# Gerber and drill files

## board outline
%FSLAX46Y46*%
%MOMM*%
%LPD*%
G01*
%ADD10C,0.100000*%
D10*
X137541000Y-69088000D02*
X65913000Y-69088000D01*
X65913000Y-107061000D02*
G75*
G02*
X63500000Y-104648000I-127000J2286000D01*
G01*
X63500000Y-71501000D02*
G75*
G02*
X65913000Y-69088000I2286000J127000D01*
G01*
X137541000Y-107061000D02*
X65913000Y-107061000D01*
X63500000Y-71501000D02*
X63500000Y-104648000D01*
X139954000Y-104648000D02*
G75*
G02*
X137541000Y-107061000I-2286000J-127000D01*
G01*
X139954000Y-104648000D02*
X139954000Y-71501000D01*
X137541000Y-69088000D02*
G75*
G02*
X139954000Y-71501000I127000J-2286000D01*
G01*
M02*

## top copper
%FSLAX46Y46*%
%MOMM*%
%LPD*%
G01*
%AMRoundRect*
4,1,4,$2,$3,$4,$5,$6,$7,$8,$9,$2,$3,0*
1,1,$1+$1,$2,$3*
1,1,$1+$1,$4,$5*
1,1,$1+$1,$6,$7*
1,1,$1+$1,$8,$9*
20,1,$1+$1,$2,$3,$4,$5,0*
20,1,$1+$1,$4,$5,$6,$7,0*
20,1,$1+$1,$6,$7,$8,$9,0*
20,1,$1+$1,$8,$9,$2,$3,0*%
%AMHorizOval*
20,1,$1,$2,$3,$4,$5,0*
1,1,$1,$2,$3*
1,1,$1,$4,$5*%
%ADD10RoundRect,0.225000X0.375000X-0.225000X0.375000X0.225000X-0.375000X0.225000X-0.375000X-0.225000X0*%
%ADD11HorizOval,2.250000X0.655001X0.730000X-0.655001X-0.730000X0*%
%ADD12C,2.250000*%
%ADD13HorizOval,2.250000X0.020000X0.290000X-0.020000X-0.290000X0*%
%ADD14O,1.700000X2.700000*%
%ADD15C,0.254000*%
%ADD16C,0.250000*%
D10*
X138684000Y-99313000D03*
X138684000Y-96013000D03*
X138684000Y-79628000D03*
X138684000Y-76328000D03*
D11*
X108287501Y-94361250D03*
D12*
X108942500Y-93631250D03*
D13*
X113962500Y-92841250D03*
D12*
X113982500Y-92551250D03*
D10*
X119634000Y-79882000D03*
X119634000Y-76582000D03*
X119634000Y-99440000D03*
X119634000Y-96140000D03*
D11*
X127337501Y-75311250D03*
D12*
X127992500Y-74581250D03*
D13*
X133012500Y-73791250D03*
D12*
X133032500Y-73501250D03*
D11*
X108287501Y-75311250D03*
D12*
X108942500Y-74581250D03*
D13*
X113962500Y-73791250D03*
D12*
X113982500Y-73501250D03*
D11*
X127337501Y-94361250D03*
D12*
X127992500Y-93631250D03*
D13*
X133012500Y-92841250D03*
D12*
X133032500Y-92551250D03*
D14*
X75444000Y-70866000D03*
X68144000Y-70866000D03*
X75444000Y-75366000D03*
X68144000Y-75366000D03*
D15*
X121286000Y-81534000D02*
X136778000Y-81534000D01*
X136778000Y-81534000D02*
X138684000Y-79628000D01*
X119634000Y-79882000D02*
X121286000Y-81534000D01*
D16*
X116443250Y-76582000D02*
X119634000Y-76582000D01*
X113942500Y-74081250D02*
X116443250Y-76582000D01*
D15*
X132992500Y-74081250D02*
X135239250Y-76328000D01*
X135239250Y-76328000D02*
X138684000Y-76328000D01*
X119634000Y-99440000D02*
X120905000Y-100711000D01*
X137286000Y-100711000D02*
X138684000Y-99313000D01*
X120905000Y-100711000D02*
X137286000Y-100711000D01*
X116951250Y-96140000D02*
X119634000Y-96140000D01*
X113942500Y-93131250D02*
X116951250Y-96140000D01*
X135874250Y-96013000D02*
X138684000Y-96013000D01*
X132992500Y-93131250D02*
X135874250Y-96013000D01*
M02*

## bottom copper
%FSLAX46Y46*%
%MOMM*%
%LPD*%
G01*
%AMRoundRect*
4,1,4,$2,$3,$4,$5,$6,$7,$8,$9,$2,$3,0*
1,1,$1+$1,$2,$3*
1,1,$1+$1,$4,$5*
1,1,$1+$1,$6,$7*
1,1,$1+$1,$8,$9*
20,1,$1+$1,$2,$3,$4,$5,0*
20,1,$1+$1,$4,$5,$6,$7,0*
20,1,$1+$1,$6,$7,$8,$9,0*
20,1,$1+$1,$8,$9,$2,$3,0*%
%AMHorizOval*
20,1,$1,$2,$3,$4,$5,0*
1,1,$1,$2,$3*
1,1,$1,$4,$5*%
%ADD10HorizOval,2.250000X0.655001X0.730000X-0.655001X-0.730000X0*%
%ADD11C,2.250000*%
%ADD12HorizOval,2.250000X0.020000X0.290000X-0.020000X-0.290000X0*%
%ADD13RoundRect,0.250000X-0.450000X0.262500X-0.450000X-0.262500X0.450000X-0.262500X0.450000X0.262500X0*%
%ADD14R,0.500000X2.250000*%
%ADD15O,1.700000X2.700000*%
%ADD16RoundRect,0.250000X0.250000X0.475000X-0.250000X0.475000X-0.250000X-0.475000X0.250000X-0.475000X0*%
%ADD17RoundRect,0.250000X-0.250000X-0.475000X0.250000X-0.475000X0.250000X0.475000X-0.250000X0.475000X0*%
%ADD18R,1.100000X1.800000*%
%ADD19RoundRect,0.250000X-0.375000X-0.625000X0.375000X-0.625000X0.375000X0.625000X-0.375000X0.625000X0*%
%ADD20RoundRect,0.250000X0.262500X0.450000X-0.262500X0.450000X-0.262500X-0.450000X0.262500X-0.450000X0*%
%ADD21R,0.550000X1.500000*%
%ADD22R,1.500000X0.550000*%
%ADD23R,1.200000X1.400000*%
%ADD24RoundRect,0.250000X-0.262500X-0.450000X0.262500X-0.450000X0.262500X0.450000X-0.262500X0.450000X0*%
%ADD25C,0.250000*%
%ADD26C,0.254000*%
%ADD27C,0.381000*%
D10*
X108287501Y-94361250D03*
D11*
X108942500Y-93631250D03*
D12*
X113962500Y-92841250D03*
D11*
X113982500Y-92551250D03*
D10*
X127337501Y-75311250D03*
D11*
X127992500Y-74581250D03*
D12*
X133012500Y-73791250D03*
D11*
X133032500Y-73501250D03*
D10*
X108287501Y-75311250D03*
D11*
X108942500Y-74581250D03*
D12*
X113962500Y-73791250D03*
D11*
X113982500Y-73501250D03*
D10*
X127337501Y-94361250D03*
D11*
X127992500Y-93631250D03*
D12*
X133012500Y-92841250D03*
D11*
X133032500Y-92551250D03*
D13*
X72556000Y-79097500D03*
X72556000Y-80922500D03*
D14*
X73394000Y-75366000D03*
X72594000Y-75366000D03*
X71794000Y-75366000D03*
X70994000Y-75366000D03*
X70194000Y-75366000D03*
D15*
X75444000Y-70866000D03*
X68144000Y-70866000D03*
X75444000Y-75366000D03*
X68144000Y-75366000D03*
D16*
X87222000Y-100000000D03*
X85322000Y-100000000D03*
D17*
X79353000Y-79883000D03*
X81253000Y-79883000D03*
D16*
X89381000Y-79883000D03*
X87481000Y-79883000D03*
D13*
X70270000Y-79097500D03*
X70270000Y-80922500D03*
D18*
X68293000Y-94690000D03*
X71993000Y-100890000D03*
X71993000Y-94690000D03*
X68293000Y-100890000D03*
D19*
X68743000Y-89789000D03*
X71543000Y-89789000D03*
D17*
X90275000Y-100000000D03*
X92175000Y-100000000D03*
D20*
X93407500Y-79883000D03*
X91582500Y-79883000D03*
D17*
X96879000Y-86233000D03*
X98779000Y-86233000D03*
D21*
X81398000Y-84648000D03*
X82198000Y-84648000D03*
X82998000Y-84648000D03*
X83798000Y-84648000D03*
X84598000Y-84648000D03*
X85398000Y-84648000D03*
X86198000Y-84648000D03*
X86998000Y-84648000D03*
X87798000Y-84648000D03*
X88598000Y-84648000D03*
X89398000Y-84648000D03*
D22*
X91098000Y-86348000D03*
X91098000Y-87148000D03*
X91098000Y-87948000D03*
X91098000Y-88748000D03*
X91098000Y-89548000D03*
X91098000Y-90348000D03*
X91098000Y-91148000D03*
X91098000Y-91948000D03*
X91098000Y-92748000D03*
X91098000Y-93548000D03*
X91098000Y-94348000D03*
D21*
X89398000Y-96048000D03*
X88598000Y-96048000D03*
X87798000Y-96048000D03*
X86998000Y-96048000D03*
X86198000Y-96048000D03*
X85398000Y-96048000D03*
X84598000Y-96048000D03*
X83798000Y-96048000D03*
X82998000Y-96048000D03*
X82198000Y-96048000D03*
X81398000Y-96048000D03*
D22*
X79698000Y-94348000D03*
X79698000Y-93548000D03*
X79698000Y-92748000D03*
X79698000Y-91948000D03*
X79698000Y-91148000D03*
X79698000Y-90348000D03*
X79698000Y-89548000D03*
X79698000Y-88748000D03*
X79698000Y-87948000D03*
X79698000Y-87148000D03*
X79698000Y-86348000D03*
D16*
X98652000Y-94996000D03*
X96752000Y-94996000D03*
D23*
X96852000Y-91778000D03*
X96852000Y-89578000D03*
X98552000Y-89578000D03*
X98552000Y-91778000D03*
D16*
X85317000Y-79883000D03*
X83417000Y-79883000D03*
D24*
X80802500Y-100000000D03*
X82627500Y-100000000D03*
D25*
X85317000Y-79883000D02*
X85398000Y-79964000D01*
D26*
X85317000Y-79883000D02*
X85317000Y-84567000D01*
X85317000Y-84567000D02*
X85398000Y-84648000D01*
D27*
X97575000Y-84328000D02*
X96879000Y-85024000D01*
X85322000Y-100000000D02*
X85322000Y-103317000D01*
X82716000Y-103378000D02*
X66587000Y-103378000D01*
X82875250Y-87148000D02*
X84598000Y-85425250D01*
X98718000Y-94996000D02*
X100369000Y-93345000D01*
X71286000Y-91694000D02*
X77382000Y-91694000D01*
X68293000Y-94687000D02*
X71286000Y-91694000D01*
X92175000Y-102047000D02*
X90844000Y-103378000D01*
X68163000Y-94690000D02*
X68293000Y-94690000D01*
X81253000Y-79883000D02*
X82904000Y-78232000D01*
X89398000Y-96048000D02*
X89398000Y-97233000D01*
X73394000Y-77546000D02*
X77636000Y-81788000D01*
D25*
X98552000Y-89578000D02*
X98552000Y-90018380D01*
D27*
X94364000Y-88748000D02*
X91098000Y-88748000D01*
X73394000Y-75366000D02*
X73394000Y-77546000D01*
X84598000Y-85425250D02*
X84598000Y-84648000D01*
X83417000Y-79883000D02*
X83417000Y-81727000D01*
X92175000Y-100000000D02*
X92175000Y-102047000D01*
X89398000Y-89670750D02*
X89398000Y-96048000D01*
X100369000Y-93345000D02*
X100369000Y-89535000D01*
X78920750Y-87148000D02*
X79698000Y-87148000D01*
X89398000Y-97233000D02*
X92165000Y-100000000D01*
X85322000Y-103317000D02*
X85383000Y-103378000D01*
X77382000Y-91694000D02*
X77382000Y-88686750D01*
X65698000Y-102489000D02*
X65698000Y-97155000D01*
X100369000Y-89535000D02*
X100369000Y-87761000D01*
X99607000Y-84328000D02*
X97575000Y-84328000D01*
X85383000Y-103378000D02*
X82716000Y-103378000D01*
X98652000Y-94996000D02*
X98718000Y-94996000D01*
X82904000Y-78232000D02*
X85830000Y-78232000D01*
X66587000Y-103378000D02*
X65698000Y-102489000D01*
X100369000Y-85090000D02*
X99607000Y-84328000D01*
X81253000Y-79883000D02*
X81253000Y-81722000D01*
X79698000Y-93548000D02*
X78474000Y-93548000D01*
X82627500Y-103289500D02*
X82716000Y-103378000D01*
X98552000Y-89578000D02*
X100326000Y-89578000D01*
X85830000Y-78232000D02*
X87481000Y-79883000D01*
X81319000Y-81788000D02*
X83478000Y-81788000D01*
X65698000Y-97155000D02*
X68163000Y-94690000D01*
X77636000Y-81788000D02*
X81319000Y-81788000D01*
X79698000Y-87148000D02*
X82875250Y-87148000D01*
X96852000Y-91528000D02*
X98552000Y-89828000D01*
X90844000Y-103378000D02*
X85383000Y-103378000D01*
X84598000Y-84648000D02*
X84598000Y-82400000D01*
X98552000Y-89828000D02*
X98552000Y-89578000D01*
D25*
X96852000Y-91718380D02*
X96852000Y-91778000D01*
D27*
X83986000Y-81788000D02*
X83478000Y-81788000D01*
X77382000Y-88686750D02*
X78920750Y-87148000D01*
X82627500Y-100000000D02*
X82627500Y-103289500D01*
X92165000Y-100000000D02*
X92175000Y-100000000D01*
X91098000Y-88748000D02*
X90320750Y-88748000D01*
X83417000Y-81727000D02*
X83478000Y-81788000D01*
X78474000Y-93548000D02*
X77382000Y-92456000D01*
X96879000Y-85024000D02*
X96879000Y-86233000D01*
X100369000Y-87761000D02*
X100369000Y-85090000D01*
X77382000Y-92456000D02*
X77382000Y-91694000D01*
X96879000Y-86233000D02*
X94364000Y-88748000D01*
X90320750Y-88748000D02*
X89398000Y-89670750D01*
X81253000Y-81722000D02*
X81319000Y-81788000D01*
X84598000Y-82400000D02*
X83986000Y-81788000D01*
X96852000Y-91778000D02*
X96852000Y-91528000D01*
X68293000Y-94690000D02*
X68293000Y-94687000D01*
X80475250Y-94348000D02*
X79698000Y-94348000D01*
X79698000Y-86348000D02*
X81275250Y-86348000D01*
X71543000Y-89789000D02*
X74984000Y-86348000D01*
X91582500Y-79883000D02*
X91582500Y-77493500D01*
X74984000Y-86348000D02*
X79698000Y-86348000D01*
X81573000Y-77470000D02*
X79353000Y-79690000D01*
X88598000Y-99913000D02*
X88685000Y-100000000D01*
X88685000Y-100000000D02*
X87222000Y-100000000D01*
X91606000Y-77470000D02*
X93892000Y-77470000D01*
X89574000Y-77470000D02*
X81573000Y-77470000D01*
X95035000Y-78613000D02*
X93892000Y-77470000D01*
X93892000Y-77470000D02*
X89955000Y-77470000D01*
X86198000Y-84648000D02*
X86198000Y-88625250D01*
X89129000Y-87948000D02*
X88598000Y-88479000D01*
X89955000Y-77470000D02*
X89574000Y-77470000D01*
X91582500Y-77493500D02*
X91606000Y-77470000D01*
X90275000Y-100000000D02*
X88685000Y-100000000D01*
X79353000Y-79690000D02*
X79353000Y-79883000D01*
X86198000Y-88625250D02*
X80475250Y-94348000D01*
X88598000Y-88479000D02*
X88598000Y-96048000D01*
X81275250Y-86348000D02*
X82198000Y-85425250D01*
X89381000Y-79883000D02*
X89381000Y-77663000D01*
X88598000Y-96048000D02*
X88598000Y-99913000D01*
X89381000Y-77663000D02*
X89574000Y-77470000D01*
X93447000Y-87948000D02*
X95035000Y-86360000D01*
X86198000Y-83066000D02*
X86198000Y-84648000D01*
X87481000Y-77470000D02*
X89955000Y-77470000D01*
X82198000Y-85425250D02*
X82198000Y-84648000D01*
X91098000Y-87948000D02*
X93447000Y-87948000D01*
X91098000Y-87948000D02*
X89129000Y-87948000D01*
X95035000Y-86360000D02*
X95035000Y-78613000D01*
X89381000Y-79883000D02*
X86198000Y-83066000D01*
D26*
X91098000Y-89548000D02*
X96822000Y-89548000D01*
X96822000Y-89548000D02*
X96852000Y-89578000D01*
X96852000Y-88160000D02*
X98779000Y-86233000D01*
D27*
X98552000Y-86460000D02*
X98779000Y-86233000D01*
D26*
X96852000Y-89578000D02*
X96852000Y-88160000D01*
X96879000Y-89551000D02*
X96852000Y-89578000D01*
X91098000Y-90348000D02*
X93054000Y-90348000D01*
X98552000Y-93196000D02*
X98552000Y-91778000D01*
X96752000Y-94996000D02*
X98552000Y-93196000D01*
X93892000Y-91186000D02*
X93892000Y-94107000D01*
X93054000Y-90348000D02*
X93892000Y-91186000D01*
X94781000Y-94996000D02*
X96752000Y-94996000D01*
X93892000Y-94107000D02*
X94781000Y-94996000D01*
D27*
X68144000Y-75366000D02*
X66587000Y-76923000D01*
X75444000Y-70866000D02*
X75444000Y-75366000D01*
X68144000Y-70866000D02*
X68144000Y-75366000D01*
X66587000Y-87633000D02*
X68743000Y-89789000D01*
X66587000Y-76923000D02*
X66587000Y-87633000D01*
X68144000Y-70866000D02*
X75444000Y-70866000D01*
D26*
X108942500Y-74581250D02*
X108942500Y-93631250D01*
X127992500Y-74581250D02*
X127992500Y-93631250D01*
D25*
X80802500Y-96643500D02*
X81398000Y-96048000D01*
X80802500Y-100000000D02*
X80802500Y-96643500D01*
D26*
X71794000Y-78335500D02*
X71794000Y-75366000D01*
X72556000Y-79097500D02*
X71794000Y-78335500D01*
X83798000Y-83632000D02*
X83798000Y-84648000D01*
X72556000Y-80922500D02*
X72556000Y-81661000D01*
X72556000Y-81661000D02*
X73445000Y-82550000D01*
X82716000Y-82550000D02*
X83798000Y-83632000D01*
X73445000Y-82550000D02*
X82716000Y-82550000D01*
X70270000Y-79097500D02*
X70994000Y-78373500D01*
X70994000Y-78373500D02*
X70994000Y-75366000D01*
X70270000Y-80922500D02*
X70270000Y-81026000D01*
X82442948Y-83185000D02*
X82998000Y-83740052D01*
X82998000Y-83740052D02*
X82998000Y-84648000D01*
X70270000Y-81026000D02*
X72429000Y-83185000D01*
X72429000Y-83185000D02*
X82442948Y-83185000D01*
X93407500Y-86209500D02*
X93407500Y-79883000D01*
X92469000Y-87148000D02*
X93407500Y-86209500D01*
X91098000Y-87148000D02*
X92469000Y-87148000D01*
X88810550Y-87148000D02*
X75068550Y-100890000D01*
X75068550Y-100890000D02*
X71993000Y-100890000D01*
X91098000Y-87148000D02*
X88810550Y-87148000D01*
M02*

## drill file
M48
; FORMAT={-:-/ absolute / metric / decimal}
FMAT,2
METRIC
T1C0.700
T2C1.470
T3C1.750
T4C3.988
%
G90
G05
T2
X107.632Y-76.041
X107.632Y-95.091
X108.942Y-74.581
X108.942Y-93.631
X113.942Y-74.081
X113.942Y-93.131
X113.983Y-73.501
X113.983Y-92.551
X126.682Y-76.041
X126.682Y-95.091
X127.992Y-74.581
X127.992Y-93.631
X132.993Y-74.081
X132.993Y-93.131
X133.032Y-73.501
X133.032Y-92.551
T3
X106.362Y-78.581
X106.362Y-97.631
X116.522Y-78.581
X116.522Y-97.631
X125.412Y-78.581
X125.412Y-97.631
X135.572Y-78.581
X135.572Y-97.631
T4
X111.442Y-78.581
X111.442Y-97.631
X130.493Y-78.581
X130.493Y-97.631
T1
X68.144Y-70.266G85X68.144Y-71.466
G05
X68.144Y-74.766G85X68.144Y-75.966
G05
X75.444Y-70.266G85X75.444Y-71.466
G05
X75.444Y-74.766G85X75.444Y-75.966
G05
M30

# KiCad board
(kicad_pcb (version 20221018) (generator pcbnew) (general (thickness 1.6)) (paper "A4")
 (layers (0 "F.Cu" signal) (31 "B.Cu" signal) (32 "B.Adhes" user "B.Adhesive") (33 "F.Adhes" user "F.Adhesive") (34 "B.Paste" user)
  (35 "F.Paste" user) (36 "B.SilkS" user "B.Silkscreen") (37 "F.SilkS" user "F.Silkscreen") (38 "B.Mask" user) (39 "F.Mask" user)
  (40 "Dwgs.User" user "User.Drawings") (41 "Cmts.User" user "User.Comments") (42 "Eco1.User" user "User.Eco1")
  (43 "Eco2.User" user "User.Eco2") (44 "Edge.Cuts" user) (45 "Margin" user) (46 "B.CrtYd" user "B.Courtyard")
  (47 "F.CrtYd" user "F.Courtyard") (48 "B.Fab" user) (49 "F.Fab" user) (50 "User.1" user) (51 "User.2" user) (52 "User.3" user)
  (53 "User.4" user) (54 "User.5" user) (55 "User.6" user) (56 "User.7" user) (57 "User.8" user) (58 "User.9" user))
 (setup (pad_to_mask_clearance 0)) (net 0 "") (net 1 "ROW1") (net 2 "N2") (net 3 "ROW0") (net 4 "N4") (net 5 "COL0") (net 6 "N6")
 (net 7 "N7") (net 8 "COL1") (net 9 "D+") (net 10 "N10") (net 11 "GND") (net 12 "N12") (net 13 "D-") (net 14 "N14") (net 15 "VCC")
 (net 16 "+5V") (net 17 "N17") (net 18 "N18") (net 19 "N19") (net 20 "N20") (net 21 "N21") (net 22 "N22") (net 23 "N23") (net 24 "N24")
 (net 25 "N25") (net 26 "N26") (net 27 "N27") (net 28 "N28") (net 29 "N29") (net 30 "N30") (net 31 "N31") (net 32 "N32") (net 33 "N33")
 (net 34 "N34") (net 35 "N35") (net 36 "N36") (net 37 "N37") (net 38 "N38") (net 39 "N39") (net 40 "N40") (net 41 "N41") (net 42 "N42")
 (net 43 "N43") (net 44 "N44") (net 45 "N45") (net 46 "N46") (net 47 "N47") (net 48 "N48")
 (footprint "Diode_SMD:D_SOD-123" (layer "F.Cu") (at 138.684 97.663 90)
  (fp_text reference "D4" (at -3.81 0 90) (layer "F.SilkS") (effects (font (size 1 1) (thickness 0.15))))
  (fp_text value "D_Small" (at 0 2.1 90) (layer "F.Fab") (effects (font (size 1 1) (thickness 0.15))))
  (pad "1" smd roundrect (at -1.65 0 90) (size 0.9 1.2) (layers "F.Cu" "F.Paste" "F.Mask") (roundrect_rratio 0.25) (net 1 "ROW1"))
  (pad "2" smd roundrect (at 1.65 0 90) (size 0.9 1.2) (layers "F.Cu" "F.Paste" "F.Mask") (roundrect_rratio 0.25) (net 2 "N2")))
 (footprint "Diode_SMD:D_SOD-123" (layer "F.Cu") (at 138.684 77.978 90)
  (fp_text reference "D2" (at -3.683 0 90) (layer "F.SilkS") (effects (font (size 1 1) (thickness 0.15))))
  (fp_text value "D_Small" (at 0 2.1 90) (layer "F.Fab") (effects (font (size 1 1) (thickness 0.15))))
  (pad "1" smd roundrect (at -1.65 0 90) (size 0.9 1.2) (layers "F.Cu" "F.Paste" "F.Mask") (roundrect_rratio 0.25) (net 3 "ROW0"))
  (pad "2" smd roundrect (at 1.65 0 90) (size 0.9 1.2) (layers "F.Cu" "F.Paste" "F.Mask") (roundrect_rratio 0.25) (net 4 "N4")))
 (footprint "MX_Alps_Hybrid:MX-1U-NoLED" (layer "F.Cu") (at 111.4425 97.63125)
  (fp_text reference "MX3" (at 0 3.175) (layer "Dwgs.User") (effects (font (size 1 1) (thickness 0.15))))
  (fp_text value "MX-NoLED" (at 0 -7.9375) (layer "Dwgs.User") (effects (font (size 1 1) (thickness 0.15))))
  (pad "" np_thru_hole circle (at -5.08 0 48.0996) (size 1.75 1.75) (drill 1.75) (layers "*.Cu" "*.Mask"))
  (pad "" np_thru_hole circle (at 0 0) (size 3.9878 3.9878) (drill 3.9878) (layers "*.Cu" "*.Mask"))
  (pad "" np_thru_hole circle (at 5.08 0 48.0996) (size 1.75 1.75) (drill 1.75) (layers "*.Cu" "*.Mask"))
  (pad "1" thru_hole oval (at -3.81 -2.54 48.0996) (size 4.211556 2.25) (drill 1.47 (offset 0.980778 0)) (layers "*.Cu" "B.Mask")
   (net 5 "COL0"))
  (pad "1" thru_hole circle (at -2.5 -4) (size 2.25 2.25) (drill 1.47) (layers "*.Cu" "B.Mask") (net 5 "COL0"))
  (pad "2" thru_hole oval (at 2.5 -4.5 86.0548) (size 2.831378 2.25) (drill 1.47 (offset 0.290689 0)) (layers "*.Cu" "B.Mask") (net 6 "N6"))
  (pad "2" thru_hole circle (at 2.54 -5.08) (size 2.25 2.25) (drill 1.47) (layers "*.Cu" "B.Mask") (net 6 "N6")))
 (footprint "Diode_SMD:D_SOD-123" (layer "F.Cu") (at 119.634 78.232 90)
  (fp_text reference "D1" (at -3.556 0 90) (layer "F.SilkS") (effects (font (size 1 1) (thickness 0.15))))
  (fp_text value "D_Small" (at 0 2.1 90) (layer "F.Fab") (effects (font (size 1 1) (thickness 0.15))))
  (pad "1" smd roundrect (at -1.65 0 90) (size 0.9 1.2) (layers "F.Cu" "F.Paste" "F.Mask") (roundrect_rratio 0.25) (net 3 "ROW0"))
  (pad "2" smd roundrect (at 1.65 0 90) (size 0.9 1.2) (layers "F.Cu" "F.Paste" "F.Mask") (roundrect_rratio 0.25) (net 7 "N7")))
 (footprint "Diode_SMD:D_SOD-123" (layer "F.Cu") (at 119.634 97.79 90)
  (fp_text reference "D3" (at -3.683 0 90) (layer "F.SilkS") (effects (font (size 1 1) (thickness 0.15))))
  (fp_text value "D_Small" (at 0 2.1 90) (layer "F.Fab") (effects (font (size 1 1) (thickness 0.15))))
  (pad "1" smd roundrect (at -1.65 0 90) (size 0.9 1.2) (layers "F.Cu" "F.Paste" "F.Mask") (roundrect_rratio 0.25) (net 1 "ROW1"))
  (pad "2" smd roundrect (at 1.65 0 90) (size 0.9 1.2) (layers "F.Cu" "F.Paste" "F.Mask") (roundrect_rratio 0.25) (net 6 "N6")))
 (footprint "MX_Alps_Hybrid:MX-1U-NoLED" (layer "F.Cu") (at 130.4925 78.58125)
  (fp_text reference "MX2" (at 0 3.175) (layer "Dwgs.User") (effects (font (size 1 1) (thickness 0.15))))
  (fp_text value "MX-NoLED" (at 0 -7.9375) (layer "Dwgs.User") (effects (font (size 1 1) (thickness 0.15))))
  (pad "" np_thru_hole circle (at -5.08 0 48.0996) (size 1.75 1.75) (drill 1.75) (layers "*.Cu" "*.Mask"))
  (pad "" np_thru_hole circle (at 0 0) (size 3.9878 3.9878) (drill 3.9878) (layers "*.Cu" "*.Mask"))
  (pad "" np_thru_hole circle (at 5.08 0 48.0996) (size 1.75 1.75) (drill 1.75) (layers "*.Cu" "*.Mask"))
  (pad "1" thru_hole oval (at -3.81 -2.54 48.0996) (size 4.211556 2.25) (drill 1.47 (offset 0.980778 0)) (layers "*.Cu" "B.Mask")
   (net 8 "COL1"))
  (pad "1" thru_hole circle (at -2.5 -4) (size 2.25 2.25) (drill 1.47) (layers "*.Cu" "B.Mask") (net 8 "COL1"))
  (pad "2" thru_hole oval (at 2.5 -4.5 86.0548) (size 2.831378 2.25) (drill 1.47 (offset 0.290689 0)) (layers "*.Cu" "B.Mask") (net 4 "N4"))
  (pad "2" thru_hole circle (at 2.54 -5.08) (size 2.25 2.25) (drill 1.47) (layers "*.Cu" "B.Mask") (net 4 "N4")))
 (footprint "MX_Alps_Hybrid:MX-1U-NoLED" (layer "F.Cu") (at 111.4425 78.58125)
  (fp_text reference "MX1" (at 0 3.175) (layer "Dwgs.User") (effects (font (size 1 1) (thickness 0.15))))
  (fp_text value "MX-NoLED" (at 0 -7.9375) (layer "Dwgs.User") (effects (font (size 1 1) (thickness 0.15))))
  (pad "" np_thru_hole circle (at -5.08 0 48.0996) (size 1.75 1.75) (drill 1.75) (layers "*.Cu" "*.Mask"))
  (pad "" np_thru_hole circle (at 0 0) (size 3.9878 3.9878) (drill 3.9878) (layers "*.Cu" "*.Mask"))
  (pad "" np_thru_hole circle (at 5.08 0 48.0996) (size 1.75 1.75) (drill 1.75) (layers "*.Cu" "*.Mask"))
  (pad "1" thru_hole oval (at -3.81 -2.54 48.0996) (size 4.211556 2.25) (drill 1.47 (offset 0.980778 0)) (layers "*.Cu" "B.Mask")
   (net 5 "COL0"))
  (pad "1" thru_hole circle (at -2.5 -4) (size 2.25 2.25) (drill 1.47) (layers "*.Cu" "B.Mask") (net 5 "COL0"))
  (pad "2" thru_hole oval (at 2.5 -4.5 86.0548) (size 2.831378 2.25) (drill 1.47 (offset 0.290689 0)) (layers "*.Cu" "B.Mask") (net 7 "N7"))
  (pad "2" thru_hole circle (at 2.54 -5.08) (size 2.25 2.25) (drill 1.47) (layers "*.Cu" "B.Mask") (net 7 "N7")))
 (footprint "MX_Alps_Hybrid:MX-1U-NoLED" (layer "F.Cu") (at 130.4925 97.63125)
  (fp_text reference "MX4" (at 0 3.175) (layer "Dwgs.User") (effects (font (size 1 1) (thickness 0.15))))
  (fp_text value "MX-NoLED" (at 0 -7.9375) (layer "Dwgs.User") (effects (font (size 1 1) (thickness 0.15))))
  (pad "" np_thru_hole circle (at -5.08 0 48.0996) (size 1.75 1.75) (drill 1.75) (layers "*.Cu" "*.Mask"))
  (pad "" np_thru_hole circle (at 0 0) (size 3.9878 3.9878) (drill 3.9878) (layers "*.Cu" "*.Mask"))
  (pad "" np_thru_hole circle (at 5.08 0 48.0996) (size 1.75 1.75) (drill 1.75) (layers "*.Cu" "*.Mask"))
  (pad "1" thru_hole oval (at -3.81 -2.54 48.0996) (size 4.211556 2.25) (drill 1.47 (offset 0.980778 0)) (layers "*.Cu" "B.Mask")
   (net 8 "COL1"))
  (pad "1" thru_hole circle (at -2.5 -4) (size 2.25 2.25) (drill 1.47) (layers "*.Cu" "B.Mask") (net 8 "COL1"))
  (pad "2" thru_hole oval (at 2.5 -4.5 86.0548) (size 2.831378 2.25) (drill 1.47 (offset 0.290689 0)) (layers "*.Cu" "B.Mask") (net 2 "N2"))
  (pad "2" thru_hole circle (at 2.54 -5.08) (size 2.25 2.25) (drill 1.47) (layers "*.Cu" "B.Mask") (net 2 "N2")))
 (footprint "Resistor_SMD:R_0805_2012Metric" (layer "B.Cu") (at 72.556 80.01 -90)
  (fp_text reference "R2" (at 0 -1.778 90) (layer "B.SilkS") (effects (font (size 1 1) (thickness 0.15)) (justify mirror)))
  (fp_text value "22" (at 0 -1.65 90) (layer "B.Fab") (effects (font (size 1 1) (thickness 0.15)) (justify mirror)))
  (pad "1" smd roundrect (at -0.9125 0 270) (size 1.025 1.4) (layers "B.Cu" "B.Paste" "B.Mask") (roundrect_rratio 0.243902) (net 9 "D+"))
  (pad "2" smd roundrect (at 0.9125 0 270) (size 1.025 1.4) (layers "B.Cu" "B.Paste" "B.Mask") (roundrect_rratio 0.243902) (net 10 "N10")))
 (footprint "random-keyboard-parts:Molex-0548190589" (layer "B.Cu") (at 71.794 70.866 -90)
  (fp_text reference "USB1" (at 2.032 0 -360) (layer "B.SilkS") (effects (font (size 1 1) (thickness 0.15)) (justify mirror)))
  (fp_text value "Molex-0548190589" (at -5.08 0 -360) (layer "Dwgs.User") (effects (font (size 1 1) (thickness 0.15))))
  (pad "1" smd rect (at 4.5 -1.6 270) (size 2.25 0.5) (layers "B.Cu" "B.Paste" "B.Mask") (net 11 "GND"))
  (pad "2" smd rect (at 4.5 -0.8 270) (size 2.25 0.5) (layers "B.Cu" "B.Paste" "B.Mask") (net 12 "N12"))
  (pad "3" smd rect (at 4.5 0 270) (size 2.25 0.5) (layers "B.Cu" "B.Paste" "B.Mask") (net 9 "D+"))
  (pad "4" smd rect (at 4.5 0.8 270) (size 2.25 0.5) (layers "B.Cu" "B.Paste" "B.Mask") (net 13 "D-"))
  (pad "5" smd rect (at 4.5 1.6 270) (size 2.25 0.5) (layers "B.Cu" "B.Paste" "B.Mask") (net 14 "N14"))
  (pad "6" thru_hole oval (at 0 -3.65 270) (size 2.7 1.7) (drill oval 1.9 0.7) (layers "*.Cu" "*.Mask") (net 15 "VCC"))
  (pad "6" thru_hole oval (at 0 3.65 270) (size 2.7 1.7) (drill oval 1.9 0.7) (layers "*.Cu" "*.Mask") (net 15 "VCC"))
  (pad "6" thru_hole oval (at 4.5 -3.65 270) (size 2.7 1.7) (drill oval 1.9 0.7) (layers "*.Cu" "*.Mask") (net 15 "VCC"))
  (pad "6" thru_hole oval (at 4.5 3.65 270) (size 2.7 1.7) (drill oval 1.9 0.7) (layers "*.Cu" "*.Mask") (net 15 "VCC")))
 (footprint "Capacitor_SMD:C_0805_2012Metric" (layer "B.Cu") (at 86.272 100 180)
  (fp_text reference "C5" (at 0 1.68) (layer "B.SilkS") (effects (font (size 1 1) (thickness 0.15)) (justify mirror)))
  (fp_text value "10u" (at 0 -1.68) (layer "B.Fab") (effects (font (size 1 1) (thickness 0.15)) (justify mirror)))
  (pad "1" smd roundrect (at -0.95 0 180) (size 1 1.45) (layers "B.Cu" "B.Paste" "B.Mask") (roundrect_rratio 0.25) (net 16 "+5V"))
  (pad "2" smd roundrect (at 0.95 0 180) (size 1 1.45) (layers "B.Cu" "B.Paste" "B.Mask") (roundrect_rratio 0.25) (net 11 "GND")))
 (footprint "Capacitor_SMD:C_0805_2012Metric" (layer "B.Cu") (at 80.303 79.883)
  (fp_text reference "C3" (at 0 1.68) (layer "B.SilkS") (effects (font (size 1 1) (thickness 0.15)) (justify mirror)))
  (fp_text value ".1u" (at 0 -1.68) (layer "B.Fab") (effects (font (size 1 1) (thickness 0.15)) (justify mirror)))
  (pad "1" smd roundrect (at -0.95 0) (size 1 1.45) (layers "B.Cu" "B.Paste" "B.Mask") (roundrect_rratio 0.25) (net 16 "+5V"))
  (pad "2" smd roundrect (at 0.95 0) (size 1 1.45) (layers "B.Cu" "B.Paste" "B.Mask") (roundrect_rratio 0.25) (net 11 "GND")))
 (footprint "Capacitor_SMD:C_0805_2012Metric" (layer "B.Cu") (at 88.431 79.883 180)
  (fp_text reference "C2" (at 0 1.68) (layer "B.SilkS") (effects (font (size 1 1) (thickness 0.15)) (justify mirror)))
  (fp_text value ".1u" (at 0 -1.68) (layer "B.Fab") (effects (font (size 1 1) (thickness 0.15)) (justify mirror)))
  (pad "1" smd roundrect (at -0.95 0 180) (size 1 1.45) (layers "B.Cu" "B.Paste" "B.Mask") (roundrect_rratio 0.25) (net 16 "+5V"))
  (pad "2" smd roundrect (at 0.95 0 180) (size 1 1.45) (layers "B.Cu" "B.Paste" "B.Mask") (roundrect_rratio 0.25) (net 11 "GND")))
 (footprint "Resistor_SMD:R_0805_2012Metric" (layer "B.Cu") (at 70.27 80.01 -90)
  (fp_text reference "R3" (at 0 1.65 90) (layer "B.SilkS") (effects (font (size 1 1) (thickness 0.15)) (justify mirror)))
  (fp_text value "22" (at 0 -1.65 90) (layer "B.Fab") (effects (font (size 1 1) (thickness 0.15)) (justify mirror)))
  (pad "1" smd roundrect (at -0.9125 0 270) (size 1.025 1.4) (layers "B.Cu" "B.Paste" "B.Mask") (roundrect_rratio 0.243902) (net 13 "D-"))
  (pad "2" smd roundrect (at 0.9125 0 270) (size 1.025 1.4) (layers "B.Cu" "B.Paste" "B.Mask") (roundrect_rratio 0.243902) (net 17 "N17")))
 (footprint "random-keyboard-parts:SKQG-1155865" (layer "B.Cu") (at 70.143 97.79 90)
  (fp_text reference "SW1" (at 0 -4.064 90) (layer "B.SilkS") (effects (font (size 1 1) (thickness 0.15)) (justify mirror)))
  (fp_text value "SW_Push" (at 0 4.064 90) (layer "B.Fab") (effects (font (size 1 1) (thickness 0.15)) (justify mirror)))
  (pad "1" smd rect (at 3.1 -1.85 90) (size 1.8 1.1) (layers "B.Cu" "B.Paste" "B.Mask") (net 11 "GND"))
  (pad "2" smd rect (at -3.1 1.85 90) (size 1.8 1.1) (layers "B.Cu" "B.Paste" "B.Mask") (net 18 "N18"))
  (pad "3" smd rect (at 3.1 1.85 90) (size 1.8 1.1) (layers "B.Cu" "B.Paste" "B.Mask"))
  (pad "4" smd rect (at -3.1 -1.85 90) (size 1.8 1.1) (layers "B.Cu" "B.Paste" "B.Mask")))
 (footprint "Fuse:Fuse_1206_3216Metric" (layer "B.Cu") (at 70.143 89.789)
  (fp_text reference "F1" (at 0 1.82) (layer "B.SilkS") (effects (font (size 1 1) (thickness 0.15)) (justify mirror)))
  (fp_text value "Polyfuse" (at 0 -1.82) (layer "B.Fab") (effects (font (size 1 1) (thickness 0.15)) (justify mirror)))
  (pad "1" smd roundrect (at -1.4 0) (size 1.25 1.75) (layers "B.Cu" "B.Paste" "B.Mask") (roundrect_rratio 0.2) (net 15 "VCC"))
  (pad "2" smd roundrect (at 1.4 0) (size 1.25 1.75) (layers "B.Cu" "B.Paste" "B.Mask") (roundrect_rratio 0.2) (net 16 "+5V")))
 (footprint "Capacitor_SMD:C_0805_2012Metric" (layer "B.Cu") (at 91.225 100)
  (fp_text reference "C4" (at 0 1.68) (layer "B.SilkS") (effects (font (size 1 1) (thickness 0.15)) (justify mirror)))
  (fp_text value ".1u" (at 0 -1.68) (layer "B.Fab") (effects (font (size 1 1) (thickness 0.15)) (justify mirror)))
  (pad "1" smd roundrect (at -0.95 0) (size 1 1.45) (layers "B.Cu" "B.Paste" "B.Mask") (roundrect_rratio 0.25) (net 16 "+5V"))
  (pad "2" smd roundrect (at 0.95 0) (size 1 1.45) (layers "B.Cu" "B.Paste" "B.Mask") (roundrect_rratio 0.25) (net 11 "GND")))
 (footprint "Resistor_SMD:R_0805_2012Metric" (layer "B.Cu") (at 92.495 79.883 180)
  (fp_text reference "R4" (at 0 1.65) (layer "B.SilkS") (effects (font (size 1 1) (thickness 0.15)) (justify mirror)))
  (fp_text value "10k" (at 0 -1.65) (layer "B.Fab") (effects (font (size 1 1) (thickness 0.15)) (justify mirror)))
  (pad "1" smd roundrect (at -0.9125 0 180) (size 1.025 1.4) (layers "B.Cu" "B.Paste" "B.Mask") (roundrect_rratio 0.243902) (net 18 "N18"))
  (pad "2" smd roundrect (at 0.9125 0 180) (size 1.025 1.4) (layers "B.Cu" "B.Paste" "B.Mask") (roundrect_rratio 0.243902) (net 16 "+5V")))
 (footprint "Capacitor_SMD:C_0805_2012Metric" (layer "B.Cu") (at 97.829 86.233)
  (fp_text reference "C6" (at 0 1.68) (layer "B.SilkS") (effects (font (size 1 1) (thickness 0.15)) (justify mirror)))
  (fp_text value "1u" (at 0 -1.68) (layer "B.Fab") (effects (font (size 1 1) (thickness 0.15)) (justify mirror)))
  (pad "1" smd roundrect (at -0.95 0) (size 1 1.45) (layers "B.Cu" "B.Paste" "B.Mask") (roundrect_rratio 0.25) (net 11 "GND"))
  (pad "2" smd roundrect (at 0.95 0) (size 1 1.45) (layers "B.Cu" "B.Paste" "B.Mask") (roundrect_rratio 0.25) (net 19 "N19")))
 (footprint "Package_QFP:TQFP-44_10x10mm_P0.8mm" (layer "B.Cu") (at 85.398 90.348 -90)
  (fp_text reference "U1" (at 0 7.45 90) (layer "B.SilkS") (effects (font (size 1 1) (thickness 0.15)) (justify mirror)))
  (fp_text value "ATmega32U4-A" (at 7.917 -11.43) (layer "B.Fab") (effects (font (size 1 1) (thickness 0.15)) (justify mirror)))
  (pad "1" smd rect (at -5.7 4 270) (size 1.5 0.55) (layers "B.Cu" "B.Paste" "B.Mask") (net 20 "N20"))
  (pad "2" smd rect (at -5.7 3.2 270) (size 1.5 0.55) (layers "B.Cu" "B.Paste" "B.Mask") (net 16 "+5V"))
  (pad "3" smd rect (at -5.7 2.4 270) (size 1.5 0.55) (layers "B.Cu" "B.Paste" "B.Mask") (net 17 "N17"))
  (pad "4" smd rect (at -5.7 1.6 270) (size 1.5 0.55) (layers "B.Cu" "B.Paste" "B.Mask") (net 10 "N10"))
  (pad "5" smd rect (at -5.7 0.8 270) (size 1.5 0.55) (layers "B.Cu" "B.Paste" "B.Mask") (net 11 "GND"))
  (pad "6" smd rect (at -5.7 0 270) (size 1.5 0.55) (layers "B.Cu" "B.Paste" "B.Mask") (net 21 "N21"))
  (pad "7" smd rect (at -5.7 -0.8 270) (size 1.5 0.55) (layers "B.Cu" "B.Paste" "B.Mask") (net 16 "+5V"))
  (pad "8" smd rect (at -5.7 -1.6 270) (size 1.5 0.55) (layers "B.Cu" "B.Paste" "B.Mask") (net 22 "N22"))
  (pad "9" smd rect (at -5.7 -2.4 270) (size 1.5 0.55) (layers "B.Cu" "B.Paste" "B.Mask") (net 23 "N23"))
  (pad "10" smd rect (at -5.7 -3.2 270) (size 1.5 0.55) (layers "B.Cu" "B.Paste" "B.Mask") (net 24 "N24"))
  (pad "11" smd rect (at -5.7 -4 270) (size 1.5 0.55) (layers "B.Cu" "B.Paste" "B.Mask") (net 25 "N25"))
  (pad "12" smd rect (at -4 -5.7 180) (size 1.5 0.55) (layers "B.Cu" "B.Paste" "B.Mask") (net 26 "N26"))
  (pad "13" smd rect (at -3.2 -5.7 180) (size 1.5 0.55) (layers "B.Cu" "B.Paste" "B.Mask") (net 18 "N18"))
  (pad "14" smd rect (at -2.4 -5.7 180) (size 1.5 0.55) (layers "B.Cu" "B.Paste" "B.Mask") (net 16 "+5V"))
  (pad "15" smd rect (at -1.6 -5.7 180) (size 1.5 0.55) (layers "B.Cu" "B.Paste" "B.Mask") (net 11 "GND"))
  (pad "16" smd rect (at -0.8 -5.7 180) (size 1.5 0.55) (layers "B.Cu" "B.Paste" "B.Mask") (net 19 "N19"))
  (pad "17" smd rect (at 0 -5.7 180) (size 1.5 0.55) (layers "B.Cu" "B.Paste" "B.Mask") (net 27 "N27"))
  (pad "18" smd rect (at 0.8 -5.7 180) (size 1.5 0.55) (layers "B.Cu" "B.Paste" "B.Mask") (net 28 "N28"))
  (pad "19" smd rect (at 1.6 -5.7 180) (size 1.5 0.55) (layers "B.Cu" "B.Paste" "B.Mask") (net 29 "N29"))
  (pad "20" smd rect (at 2.4 -5.7 180) (size 1.5 0.55) (layers "B.Cu" "B.Paste" "B.Mask") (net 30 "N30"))
  (pad "21" smd rect (at 3.2 -5.7 180) (size 1.5 0.55) (layers "B.Cu" "B.Paste" "B.Mask") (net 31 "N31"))
  (pad "22" smd rect (at 4 -5.7 180) (size 1.5 0.55) (layers "B.Cu" "B.Paste" "B.Mask") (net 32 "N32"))
  (pad "23" smd rect (at 5.7 -4 270) (size 1.5 0.55) (layers "B.Cu" "B.Paste" "B.Mask") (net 11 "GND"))
  (pad "24" smd rect (at 5.7 -3.2 270) (size 1.5 0.55) (layers "B.Cu" "B.Paste" "B.Mask") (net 16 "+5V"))
  (pad "25" smd rect (at 5.7 -2.4 270) (size 1.5 0.55) (layers "B.Cu" "B.Paste" "B.Mask") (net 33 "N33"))
  (pad "26" smd rect (at 5.7 -1.6 270) (size 1.5 0.55) (layers "B.Cu" "B.Paste" "B.Mask") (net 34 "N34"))
  (pad "27" smd rect (at 5.7 -0.8 270) (size 1.5 0.55) (layers "B.Cu" "B.Paste" "B.Mask") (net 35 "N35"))
  (pad "28" smd rect (at 5.7 0 270) (size 1.5 0.55) (layers "B.Cu" "B.Paste" "B.Mask") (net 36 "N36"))
  (pad "29" smd rect (at 5.7 0.8 270) (size 1.5 0.55) (layers "B.Cu" "B.Paste" "B.Mask") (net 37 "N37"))
  (pad "30" smd rect (at 5.7 1.6 270) (size 1.5 0.55) (layers "B.Cu" "B.Paste" "B.Mask") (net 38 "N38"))
  (pad "31" smd rect (at 5.7 2.4 270) (size 1.5 0.55) (layers "B.Cu" "B.Paste" "B.Mask") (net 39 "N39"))
  (pad "32" smd rect (at 5.7 3.2 270) (size 1.5 0.55) (layers "B.Cu" "B.Paste" "B.Mask") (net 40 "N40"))
  (pad "33" smd rect (at 5.7 4 270) (size 1.5 0.55) (layers "B.Cu" "B.Paste" "B.Mask") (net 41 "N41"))
  (pad "34" smd rect (at 4 5.7 180) (size 1.5 0.55) (layers "B.Cu" "B.Paste" "B.Mask") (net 16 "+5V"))
  (pad "35" smd rect (at 3.2 5.7 180) (size 1.5 0.55) (layers "B.Cu" "B.Paste" "B.Mask") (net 11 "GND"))
  (pad "36" smd rect (at 2.4 5.7 180) (size 1.5 0.55) (layers "B.Cu" "B.Paste" "B.Mask") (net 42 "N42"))
  (pad "37" smd rect (at 1.6 5.7 180) (size 1.5 0.55) (layers "B.Cu" "B.Paste" "B.Mask") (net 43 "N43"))
  (pad "38" smd rect (at 0.8 5.7 180) (size 1.5 0.55) (layers "B.Cu" "B.Paste" "B.Mask") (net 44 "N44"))
  (pad "39" smd rect (at 0 5.7 180) (size 1.5 0.55) (layers "B.Cu" "B.Paste" "B.Mask") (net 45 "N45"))
  (pad "40" smd rect (at -0.8 5.7 180) (size 1.5 0.55) (layers "B.Cu" "B.Paste" "B.Mask") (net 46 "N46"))
  (pad "41" smd rect (at -1.6 5.7 180) (size 1.5 0.55) (layers "B.Cu" "B.Paste" "B.Mask") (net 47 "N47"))
  (pad "42" smd rect (at -2.4 5.7 180) (size 1.5 0.55) (layers "B.Cu" "B.Paste" "B.Mask") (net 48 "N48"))
  (pad "43" smd rect (at -3.2 5.7 180) (size 1.5 0.55) (layers "B.Cu" "B.Paste" "B.Mask") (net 11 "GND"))
  (pad "44" smd rect (at -4 5.7 180) (size 1.5 0.55) (layers "B.Cu" "B.Paste" "B.Mask") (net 16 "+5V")))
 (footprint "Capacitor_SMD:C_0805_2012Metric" (layer "B.Cu") (at 97.702 94.996 180)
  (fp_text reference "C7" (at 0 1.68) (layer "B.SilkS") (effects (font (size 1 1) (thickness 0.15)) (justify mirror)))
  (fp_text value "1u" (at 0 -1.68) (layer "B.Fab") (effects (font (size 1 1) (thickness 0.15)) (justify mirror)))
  (pad "1" smd roundrect (at -0.95 0 180) (size 1 1.45) (layers "B.Cu" "B.Paste" "B.Mask") (roundrect_rratio 0.25) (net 11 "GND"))
  (pad "2" smd roundrect (at 0.95 0 180) (size 1 1.45) (layers "B.Cu" "B.Paste" "B.Mask") (roundrect_rratio 0.25) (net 27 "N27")))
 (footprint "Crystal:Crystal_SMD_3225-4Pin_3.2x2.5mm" (layer "B.Cu") (at 97.702 90.678 90)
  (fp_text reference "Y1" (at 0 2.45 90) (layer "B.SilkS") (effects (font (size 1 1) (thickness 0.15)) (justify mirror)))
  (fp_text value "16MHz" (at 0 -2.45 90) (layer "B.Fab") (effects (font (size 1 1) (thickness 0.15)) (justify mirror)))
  (pad "1" smd rect (at -1.1 -0.85 90) (size 1.4 1.2) (layers "B.Cu" "B.Paste" "B.Mask") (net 11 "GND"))
  (pad "2" smd rect (at 1.1 -0.85 90) (size 1.4 1.2) (layers "B.Cu" "B.Paste" "B.Mask") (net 19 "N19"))
  (pad "3" smd rect (at 1.1 0.85 90) (size 1.4 1.2) (layers "B.Cu" "B.Paste" "B.Mask") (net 11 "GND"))
  (pad "4" smd rect (at -1.1 0.85 90) (size 1.4 1.2) (layers "B.Cu" "B.Paste" "B.Mask") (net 27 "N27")))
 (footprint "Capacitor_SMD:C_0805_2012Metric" (layer "B.Cu") (at 84.367 79.883 180)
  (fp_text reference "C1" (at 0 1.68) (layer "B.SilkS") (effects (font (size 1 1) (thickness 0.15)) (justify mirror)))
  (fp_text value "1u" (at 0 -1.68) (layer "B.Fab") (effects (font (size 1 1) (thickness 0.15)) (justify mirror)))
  (pad "1" smd roundrect (at -0.95 0 180) (size 1 1.45) (layers "B.Cu" "B.Paste" "B.Mask") (roundrect_rratio 0.25) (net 21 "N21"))
  (pad "2" smd roundrect (at 0.95 0 180) (size 1 1.45) (layers "B.Cu" "B.Paste" "B.Mask") (roundrect_rratio 0.25) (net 11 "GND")))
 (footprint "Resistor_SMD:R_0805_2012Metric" (layer "B.Cu") (at 81.715 100)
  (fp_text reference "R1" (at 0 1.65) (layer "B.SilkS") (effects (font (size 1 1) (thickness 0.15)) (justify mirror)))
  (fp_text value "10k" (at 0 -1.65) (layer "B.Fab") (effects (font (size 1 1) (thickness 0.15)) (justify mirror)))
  (pad "1" smd roundrect (at -0.9125 0) (size 1.025 1.4) (layers "B.Cu" "B.Paste" "B.Mask") (roundrect_rratio 0.243902) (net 41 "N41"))
  (pad "2" smd roundrect (at 0.9125 0) (size 1.025 1.4) (layers "B.Cu" "B.Paste" "B.Mask") (roundrect_rratio 0.243902) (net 11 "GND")))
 (gr_line (start 137.541 69.088) (end 65.913 69.088) (stroke (width 0.1) (type default)) (layer "Edge.Cuts"))
 (gr_arc (start 65.913 107.061) (mid 64.167061 106.393939) (end 63.5 104.648) (stroke (width 0.1) (type default)) (layer "Edge.Cuts"))
 (gr_arc (start 63.5 71.501) (mid 64.167061 69.755061) (end 65.913 69.088) (stroke (width 0.1) (type default)) (layer "Edge.Cuts"))
 (gr_line (start 137.541 107.061) (end 65.913 107.061) (stroke (width 0.1) (type default)) (layer "Edge.Cuts"))
 (gr_line (start 63.5 71.501) (end 63.5 104.648) (stroke (width 0.1) (type default)) (layer "Edge.Cuts"))
 (gr_arc (start 139.954 104.648) (mid 139.286939 106.393939) (end 137.541 107.061) (stroke (width 0.1) (type default)) (layer "Edge.Cuts"))
 (gr_line (start 139.954 104.648) (end 139.954 71.501) (stroke (width 0.1) (type default)) (layer "Edge.Cuts"))
 (gr_arc (start 137.541 69.088) (mid 139.286939 69.755061) (end 139.954 71.501) (stroke (width 0.1) (type default)) (layer "Edge.Cuts"))
 (segment (start 85.317 79.883) (end 85.398 79.964) (width 0.25) (layer "B.Cu") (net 21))
 (segment (start 85.317 79.883) (end 85.317 84.567) (width 0.254) (layer "B.Cu") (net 21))
 (segment (start 85.317 84.567) (end 85.398 84.648) (width 0.254) (layer "B.Cu") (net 21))
 (segment (start 97.575 84.328) (end 96.879 85.024) (width 0.381) (layer "B.Cu") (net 11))
 (segment (start 85.322 100) (end 85.322 103.317) (width 0.381) (layer "B.Cu") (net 11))
 (segment (start 82.716 103.378) (end 66.587 103.378) (width 0.381) (layer "B.Cu") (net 11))
 (segment (start 82.87525 87.148) (end 84.598 85.42525) (width 0.381) (layer "B.Cu") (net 11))
 (segment (start 98.718 94.996) (end 100.369 93.345) (width 0.381) (layer "B.Cu") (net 11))
 (segment (start 71.286 91.694) (end 77.382 91.694) (width 0.381) (layer "B.Cu") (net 11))
 (segment (start 68.293 94.687) (end 71.286 91.694) (width 0.381) (layer "B.Cu") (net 11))
 (segment (start 92.175 102.047) (end 90.844 103.378) (width 0.381) (layer "B.Cu") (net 11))
 (segment (start 68.163 94.69) (end 68.293 94.69) (width 0.381) (layer "B.Cu") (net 11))
 (segment (start 81.253 79.883) (end 82.904 78.232) (width 0.381) (layer "B.Cu") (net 11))
 (segment (start 89.398 96.048) (end 89.398 97.233) (width 0.381) (layer "B.Cu") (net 11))
 (segment (start 73.394 77.546) (end 77.636 81.788) (width 0.381) (layer "B.Cu") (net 11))
 (segment (start 98.552 89.578) (end 98.552 90.01838) (width 0.25) (layer "B.Cu") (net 11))
 (segment (start 94.364 88.748) (end 91.098 88.748) (width 0.381) (layer "B.Cu") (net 11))
 (segment (start 73.394 75.366) (end 73.394 77.546) (width 0.381) (layer "B.Cu") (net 11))
 (segment (start 84.598 85.42525) (end 84.598 84.648) (width 0.381) (layer "B.Cu") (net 11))
 (segment (start 83.417 79.883) (end 83.417 81.727) (width 0.381) (layer "B.Cu") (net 11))
 (segment (start 92.175 100) (end 92.175 102.047) (width 0.381) (layer "B.Cu") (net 11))
 (segment (start 89.398 89.67075) (end 89.398 96.048) (width 0.381) (layer "B.Cu") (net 11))
 (segment (start 100.369 93.345) (end 100.369 89.535) (width 0.381) (layer "B.Cu") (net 11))
 (segment (start 78.92075 87.148) (end 79.698 87.148) (width 0.381) (layer "B.Cu") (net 11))
 (segment (start 89.398 97.233) (end 92.165 100) (width 0.381) (layer "B.Cu") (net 11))
 (segment (start 85.322 103.317) (end 85.383 103.378) (width 0.381) (layer "B.Cu") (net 11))
 (segment (start 77.382 91.694) (end 77.382 88.68675) (width 0.381) (layer "B.Cu") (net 11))
 (segment (start 65.698 102.489) (end 65.698 97.155) (width 0.381) (layer "B.Cu") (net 11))
 (segment (start 100.369 89.535) (end 100.369 87.761) (width 0.381) (layer "B.Cu") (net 11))
 (segment (start 99.607 84.328) (end 97.575 84.328) (width 0.381) (layer "B.Cu") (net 11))
 (segment (start 85.383 103.378) (end 82.716 103.378) (width 0.381) (layer "B.Cu") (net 11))
 (segment (start 98.652 94.996) (end 98.718 94.996) (width 0.381) (layer "B.Cu") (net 11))
 (segment (start 82.904 78.232) (end 85.83 78.232) (width 0.381) (layer "B.Cu") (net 11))
 (segment (start 66.587 103.378) (end 65.698 102.489) (width 0.381) (layer "B.Cu") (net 11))
 (segment (start 100.369 85.09) (end 99.607 84.328) (width 0.381) (layer "B.Cu") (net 11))
 (segment (start 81.253 79.883) (end 81.253 81.722) (width 0.381) (layer "B.Cu") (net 11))
 (segment (start 79.698 93.548) (end 78.474 93.548) (width 0.381) (layer "B.Cu") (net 11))
 (segment (start 82.6275 103.2895) (end 82.716 103.378) (width 0.381) (layer "B.Cu") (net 11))
 (segment (start 98.552 89.578) (end 100.326 89.578) (width 0.381) (layer "B.Cu") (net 11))
 (segment (start 85.83 78.232) (end 87.481 79.883) (width 0.381) (layer "B.Cu") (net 11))
 (segment (start 81.319 81.788) (end 83.478 81.788) (width 0.381) (layer "B.Cu") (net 11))
 (segment (start 65.698 97.155) (end 68.163 94.69) (width 0.381) (layer "B.Cu") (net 11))
 (segment (start 77.636 81.788) (end 81.319 81.788) (width 0.381) (layer "B.Cu") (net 11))
 (segment (start 79.698 87.148) (end 82.87525 87.148) (width 0.381) (layer "B.Cu") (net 11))
 (segment (start 96.852 91.528) (end 98.552 89.828) (width 0.381) (layer "B.Cu") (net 11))
 (segment (start 90.844 103.378) (end 85.383 103.378) (width 0.381) (layer "B.Cu") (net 11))
 (segment (start 84.598 84.648) (end 84.598 82.4) (width 0.381) (layer "B.Cu") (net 11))
 (segment (start 98.552 89.828) (end 98.552 89.578) (width 0.381) (layer "B.Cu") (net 11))
 (segment (start 96.852 91.71838) (end 96.852 91.778) (width 0.25) (layer "B.Cu") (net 11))
 (segment (start 83.986 81.788) (end 83.478 81.788) (width 0.381) (layer "B.Cu") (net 11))
 (segment (start 77.382 88.68675) (end 78.92075 87.148) (width 0.381) (layer "B.Cu") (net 11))
 (segment (start 82.6275 100) (end 82.6275 103.2895) (width 0.381) (layer "B.Cu") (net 11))
 (segment (start 92.165 100) (end 92.175 100) (width 0.381) (layer "B.Cu") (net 11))
 (segment (start 91.098 88.748) (end 90.32075 88.748) (width 0.381) (layer "B.Cu") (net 11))
 (segment (start 83.417 81.727) (end 83.478 81.788) (width 0.381) (layer "B.Cu") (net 11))
 (segment (start 78.474 93.548) (end 77.382 92.456) (width 0.381) (layer "B.Cu") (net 11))
 (segment (start 96.879 85.024) (end 96.879 86.233) (width 0.381) (layer "B.Cu") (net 11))
 (segment (start 100.369 87.761) (end 100.369 85.09) (width 0.381) (layer "B.Cu") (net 11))
 (segment (start 77.382 92.456) (end 77.382 91.694) (width 0.381) (layer "B.Cu") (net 11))
 (segment (start 96.879 86.233) (end 94.364 88.748) (width 0.381) (layer "B.Cu") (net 11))
 (segment (start 90.32075 88.748) (end 89.398 89.67075) (width 0.381) (layer "B.Cu") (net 11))
 (segment (start 81.253 81.722) (end 81.319 81.788) (width 0.381) (layer "B.Cu") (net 11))
 (segment (start 84.598 82.4) (end 83.986 81.788) (width 0.381) (layer "B.Cu") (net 11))
 (segment (start 96.852 91.778) (end 96.852 91.528) (width 0.381) (layer "B.Cu") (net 11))
 (segment (start 68.293 94.69) (end 68.293 94.687) (width 0.381) (layer "B.Cu") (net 11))
 (segment (start 80.47525 94.348) (end 79.698 94.348) (width 0.381) (layer "B.Cu") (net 16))
 (segment (start 79.698 86.348) (end 81.27525 86.348) (width 0.381) (layer "B.Cu") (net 16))
 (segment (start 71.543 89.789) (end 74.984 86.348) (width 0.381) (layer "B.Cu") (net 16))
 (segment (start 91.5825 79.883) (end 91.5825 77.4935) (width 0.381) (layer "B.Cu") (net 16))
 (segment (start 74.984 86.348) (end 79.698 86.348) (width 0.381) (layer "B.Cu") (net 16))
 (segment (start 81.573 77.47) (end 79.353 79.69) (width 0.381) (layer "B.Cu") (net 16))
 (segment (start 88.598 99.913) (end 88.685 100) (width 0.381) (layer "B.Cu") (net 16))
 (segment (start 88.685 100) (end 87.222 100) (width 0.381) (layer "B.Cu") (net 16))
 (segment (start 91.606 77.47) (end 93.892 77.47) (width 0.381) (layer "B.Cu") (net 16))
 (segment (start 89.574 77.47) (end 81.573 77.47) (width 0.381) (layer "B.Cu") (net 16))
 (segment (start 95.035 78.613) (end 93.892 77.47) (width 0.381) (layer "B.Cu") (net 16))
 (segment (start 93.892 77.47) (end 89.955 77.47) (width 0.381) (layer "B.Cu") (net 16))
 (segment (start 86.198 84.648) (end 86.198 88.62525) (width 0.381) (layer "B.Cu") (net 16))
 (segment (start 89.129 87.948) (end 88.598 88.479) (width 0.381) (layer "B.Cu") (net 16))
 (segment (start 89.955 77.47) (end 89.574 77.47) (width 0.381) (layer "B.Cu") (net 16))
 (segment (start 91.5825 77.4935) (end 91.606 77.47) (width 0.381) (layer "B.Cu") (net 16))
 (segment (start 90.275 100) (end 88.685 100) (width 0.381) (layer "B.Cu") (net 16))
 (segment (start 79.353 79.69) (end 79.353 79.883) (width 0.381) (layer "B.Cu") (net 16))
 (segment (start 86.198 88.62525) (end 80.47525 94.348) (width 0.381) (layer "B.Cu") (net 16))
 (segment (start 88.598 88.479) (end 88.598 96.048) (width 0.381) (layer "B.Cu") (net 16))
 (segment (start 81.27525 86.348) (end 82.198 85.42525) (width 0.381) (layer "B.Cu") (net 16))
 (segment (start 89.381 79.883) (end 89.381 77.663) (width 0.381) (layer "B.Cu") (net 16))
 (segment (start 88.598 96.048) (end 88.598 99.913) (width 0.381) (layer "B.Cu") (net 16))
 (segment (start 89.381 77.663) (end 89.574 77.47) (width 0.381) (layer "B.Cu") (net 16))
 (segment (start 93.447 87.948) (end 95.035 86.36) (width 0.381) (layer "B.Cu") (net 16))
 (segment (start 86.198 83.066) (end 86.198 84.648) (width 0.381) (layer "B.Cu") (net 16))
 (segment (start 87.481 77.47) (end 89.955 77.47) (width 0.381) (layer "B.Cu") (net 16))
 (segment (start 82.198 85.42525) (end 82.198 84.648) (width 0.381) (layer "B.Cu") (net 16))
 (segment (start 91.098 87.948) (end 93.447 87.948) (width 0.381) (layer "B.Cu") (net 16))
 (segment (start 91.098 87.948) (end 89.129 87.948) (width 0.381) (layer "B.Cu") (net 16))
 (segment (start 95.035 86.36) (end 95.035 78.613) (width 0.381) (layer "B.Cu") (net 16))
 (segment (start 89.381 79.883) (end 86.198 83.066) (width 0.381) (layer "B.Cu") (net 16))
 (segment (start 91.098 89.548) (end 96.822 89.548) (width 0.254) (layer "B.Cu") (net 19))
 (segment (start 96.822 89.548) (end 96.852 89.578) (width 0.254) (layer "B.Cu") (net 19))
 (segment (start 96.852 88.16) (end 98.779 86.233) (width 0.254) (layer "B.Cu") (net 19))
 (segment (start 98.552 86.46) (end 98.779 86.233) (width 0.381) (layer "B.Cu") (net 19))
 (segment (start 96.852 89.578) (end 96.852 88.16) (width 0.254) (layer "B.Cu") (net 19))
 (segment (start 96.879 89.551) (end 96.852 89.578) (width 0.254) (layer "B.Cu") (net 19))
 (segment (start 91.098 90.348) (end 93.054 90.348) (width 0.254) (layer "B.Cu") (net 27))
 (segment (start 98.552 93.196) (end 98.552 91.778) (width 0.254) (layer "B.Cu") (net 27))
 (segment (start 96.752 94.996) (end 98.552 93.196) (width 0.254) (layer "B.Cu") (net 27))
 (segment (start 93.892 91.186) (end 93.892 94.107) (width 0.254) (layer "B.Cu") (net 27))
 (segment (start 93.054 90.348) (end 93.892 91.186) (width 0.254) (layer "B.Cu") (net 27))
 (segment (start 94.781 94.996) (end 96.752 94.996) (width 0.254) (layer "B.Cu") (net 27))
 (segment (start 93.892 94.107) (end 94.781 94.996) (width 0.254) (layer "B.Cu") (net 27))
 (segment (start 121.286 81.534) (end 136.778 81.534) (width 0.254) (layer "F.Cu") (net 3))
 (segment (start 136.778 81.534) (end 138.684 79.628) (width 0.254) (layer "F.Cu") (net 3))
 (segment (start 119.634 79.882) (end 121.286 81.534) (width 0.254) (layer "F.Cu") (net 3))
 (segment (start 116.44325 76.582) (end 119.634 76.582) (width 0.25) (layer "F.Cu") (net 7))
 (segment (start 113.9425 74.08125) (end 116.44325 76.582) (width 0.25) (layer "F.Cu") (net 7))
 (segment (start 132.9925 74.08125) (end 135.23925 76.328) (width 0.254) (layer "F.Cu") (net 4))
 (segment (start 135.23925 76.328) (end 138.684 76.328) (width 0.254) (layer "F.Cu") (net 4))
 (segment (start 119.634 99.44) (end 120.905 100.711) (width 0.254) (layer "F.Cu") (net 1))
 (segment (start 137.286 100.711) (end 138.684 99.313) (width 0.254) (layer "F.Cu") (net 1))
 (segment (start 120.905 100.711) (end 137.286 100.711) (width 0.254) (layer "F.Cu") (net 1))
 (segment (start 116.95125 96.14) (end 119.634 96.14) (width 0.254) (layer "F.Cu") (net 6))
 (segment (start 113.9425 93.13125) (end 116.95125 96.14) (width 0.254) (layer "F.Cu") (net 6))
 (segment (start 135.87425 96.013) (end 138.684 96.013) (width 0.254) (layer "F.Cu") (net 2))
 (segment (start 132.9925 93.13125) (end 135.87425 96.013) (width 0.254) (layer "F.Cu") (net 2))
 (segment (start 68.144 75.366) (end 66.587 76.923) (width 0.381) (layer "B.Cu") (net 15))
 (segment (start 75.444 70.866) (end 75.444 75.366) (width 0.381) (layer "B.Cu") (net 15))
 (segment (start 68.144 70.866) (end 68.144 75.366) (width 0.381) (layer "B.Cu") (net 15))
 (segment (start 66.587 87.633) (end 68.743 89.789) (width 0.381) (layer "B.Cu") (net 15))
 (segment (start 66.587 76.923) (end 66.587 87.633) (width 0.381) (layer "B.Cu") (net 15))
 (segment (start 68.144 70.866) (end 75.444 70.866) (width 0.381) (layer "B.Cu") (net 15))
 (segment (start 108.9425 74.58125) (end 108.9425 93.63125) (width 0.254) (layer "B.Cu") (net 5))
 (segment (start 127.9925 74.58125) (end 127.9925 93.63125) (width 0.254) (layer "B.Cu") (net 8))
 (segment (start 80.8025 96.6435) (end 81.398 96.048) (width 0.25) (layer "B.Cu") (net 41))
 (segment (start 80.8025 100) (end 80.8025 96.6435) (width 0.25) (layer "B.Cu") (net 41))
 (segment (start 71.794 78.3355) (end 71.794 75.366) (width 0.254) (layer "B.Cu") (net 9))
 (segment (start 72.556 79.0975) (end 71.794 78.3355) (width 0.254) (layer "B.Cu") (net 9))
 (segment (start 83.798 83.632) (end 83.798 84.648) (width 0.254) (layer "B.Cu") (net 10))
 (segment (start 72.556 80.9225) (end 72.556 81.661) (width 0.254) (layer "B.Cu") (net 10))
 (segment (start 72.556 81.661) (end 73.445 82.55) (width 0.254) (layer "B.Cu") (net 10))
 (segment (start 82.716 82.55) (end 83.798 83.632) (width 0.254) (layer "B.Cu") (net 10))
 (segment (start 73.445 82.55) (end 82.716 82.55) (width 0.254) (layer "B.Cu") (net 10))
 (segment (start 70.27 79.0975) (end 70.994 78.3735) (width 0.254) (layer "B.Cu") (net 13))
 (segment (start 70.994 78.3735) (end 70.994 75.366) (width 0.254) (layer "B.Cu") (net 13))
 (segment (start 70.27 80.9225) (end 70.27 81.026) (width 0.254) (layer "B.Cu") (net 17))
 (segment (start 82.442948 83.185) (end 82.998 83.740052) (width 0.254) (layer "B.Cu") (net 17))
 (segment (start 82.998 83.740052) (end 82.998 84.648) (width 0.254) (layer "B.Cu") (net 17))
 (segment (start 70.27 81.026) (end 72.429 83.185) (width 0.254) (layer "B.Cu") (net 17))
 (segment (start 72.429 83.185) (end 82.442948 83.185) (width 0.254) (layer "B.Cu") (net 17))
 (segment (start 93.4075 86.2095) (end 93.4075 79.883) (width 0.254) (layer "B.Cu") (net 18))
 (segment (start 92.469 87.148) (end 93.4075 86.2095) (width 0.254) (layer "B.Cu") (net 18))
 (segment (start 91.098 87.148) (end 92.469 87.148) (width 0.254) (layer "B.Cu") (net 18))
 (segment (start 88.81055 87.148) (end 75.06855 100.89) (width 0.254) (layer "B.Cu") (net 18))
 (segment (start 75.06855 100.89) (end 71.993 100.89) (width 0.254) (layer "B.Cu") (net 18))
 (segment (start 91.098 87.148) (end 88.81055 87.148) (width 0.254) (layer "B.Cu") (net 18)))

